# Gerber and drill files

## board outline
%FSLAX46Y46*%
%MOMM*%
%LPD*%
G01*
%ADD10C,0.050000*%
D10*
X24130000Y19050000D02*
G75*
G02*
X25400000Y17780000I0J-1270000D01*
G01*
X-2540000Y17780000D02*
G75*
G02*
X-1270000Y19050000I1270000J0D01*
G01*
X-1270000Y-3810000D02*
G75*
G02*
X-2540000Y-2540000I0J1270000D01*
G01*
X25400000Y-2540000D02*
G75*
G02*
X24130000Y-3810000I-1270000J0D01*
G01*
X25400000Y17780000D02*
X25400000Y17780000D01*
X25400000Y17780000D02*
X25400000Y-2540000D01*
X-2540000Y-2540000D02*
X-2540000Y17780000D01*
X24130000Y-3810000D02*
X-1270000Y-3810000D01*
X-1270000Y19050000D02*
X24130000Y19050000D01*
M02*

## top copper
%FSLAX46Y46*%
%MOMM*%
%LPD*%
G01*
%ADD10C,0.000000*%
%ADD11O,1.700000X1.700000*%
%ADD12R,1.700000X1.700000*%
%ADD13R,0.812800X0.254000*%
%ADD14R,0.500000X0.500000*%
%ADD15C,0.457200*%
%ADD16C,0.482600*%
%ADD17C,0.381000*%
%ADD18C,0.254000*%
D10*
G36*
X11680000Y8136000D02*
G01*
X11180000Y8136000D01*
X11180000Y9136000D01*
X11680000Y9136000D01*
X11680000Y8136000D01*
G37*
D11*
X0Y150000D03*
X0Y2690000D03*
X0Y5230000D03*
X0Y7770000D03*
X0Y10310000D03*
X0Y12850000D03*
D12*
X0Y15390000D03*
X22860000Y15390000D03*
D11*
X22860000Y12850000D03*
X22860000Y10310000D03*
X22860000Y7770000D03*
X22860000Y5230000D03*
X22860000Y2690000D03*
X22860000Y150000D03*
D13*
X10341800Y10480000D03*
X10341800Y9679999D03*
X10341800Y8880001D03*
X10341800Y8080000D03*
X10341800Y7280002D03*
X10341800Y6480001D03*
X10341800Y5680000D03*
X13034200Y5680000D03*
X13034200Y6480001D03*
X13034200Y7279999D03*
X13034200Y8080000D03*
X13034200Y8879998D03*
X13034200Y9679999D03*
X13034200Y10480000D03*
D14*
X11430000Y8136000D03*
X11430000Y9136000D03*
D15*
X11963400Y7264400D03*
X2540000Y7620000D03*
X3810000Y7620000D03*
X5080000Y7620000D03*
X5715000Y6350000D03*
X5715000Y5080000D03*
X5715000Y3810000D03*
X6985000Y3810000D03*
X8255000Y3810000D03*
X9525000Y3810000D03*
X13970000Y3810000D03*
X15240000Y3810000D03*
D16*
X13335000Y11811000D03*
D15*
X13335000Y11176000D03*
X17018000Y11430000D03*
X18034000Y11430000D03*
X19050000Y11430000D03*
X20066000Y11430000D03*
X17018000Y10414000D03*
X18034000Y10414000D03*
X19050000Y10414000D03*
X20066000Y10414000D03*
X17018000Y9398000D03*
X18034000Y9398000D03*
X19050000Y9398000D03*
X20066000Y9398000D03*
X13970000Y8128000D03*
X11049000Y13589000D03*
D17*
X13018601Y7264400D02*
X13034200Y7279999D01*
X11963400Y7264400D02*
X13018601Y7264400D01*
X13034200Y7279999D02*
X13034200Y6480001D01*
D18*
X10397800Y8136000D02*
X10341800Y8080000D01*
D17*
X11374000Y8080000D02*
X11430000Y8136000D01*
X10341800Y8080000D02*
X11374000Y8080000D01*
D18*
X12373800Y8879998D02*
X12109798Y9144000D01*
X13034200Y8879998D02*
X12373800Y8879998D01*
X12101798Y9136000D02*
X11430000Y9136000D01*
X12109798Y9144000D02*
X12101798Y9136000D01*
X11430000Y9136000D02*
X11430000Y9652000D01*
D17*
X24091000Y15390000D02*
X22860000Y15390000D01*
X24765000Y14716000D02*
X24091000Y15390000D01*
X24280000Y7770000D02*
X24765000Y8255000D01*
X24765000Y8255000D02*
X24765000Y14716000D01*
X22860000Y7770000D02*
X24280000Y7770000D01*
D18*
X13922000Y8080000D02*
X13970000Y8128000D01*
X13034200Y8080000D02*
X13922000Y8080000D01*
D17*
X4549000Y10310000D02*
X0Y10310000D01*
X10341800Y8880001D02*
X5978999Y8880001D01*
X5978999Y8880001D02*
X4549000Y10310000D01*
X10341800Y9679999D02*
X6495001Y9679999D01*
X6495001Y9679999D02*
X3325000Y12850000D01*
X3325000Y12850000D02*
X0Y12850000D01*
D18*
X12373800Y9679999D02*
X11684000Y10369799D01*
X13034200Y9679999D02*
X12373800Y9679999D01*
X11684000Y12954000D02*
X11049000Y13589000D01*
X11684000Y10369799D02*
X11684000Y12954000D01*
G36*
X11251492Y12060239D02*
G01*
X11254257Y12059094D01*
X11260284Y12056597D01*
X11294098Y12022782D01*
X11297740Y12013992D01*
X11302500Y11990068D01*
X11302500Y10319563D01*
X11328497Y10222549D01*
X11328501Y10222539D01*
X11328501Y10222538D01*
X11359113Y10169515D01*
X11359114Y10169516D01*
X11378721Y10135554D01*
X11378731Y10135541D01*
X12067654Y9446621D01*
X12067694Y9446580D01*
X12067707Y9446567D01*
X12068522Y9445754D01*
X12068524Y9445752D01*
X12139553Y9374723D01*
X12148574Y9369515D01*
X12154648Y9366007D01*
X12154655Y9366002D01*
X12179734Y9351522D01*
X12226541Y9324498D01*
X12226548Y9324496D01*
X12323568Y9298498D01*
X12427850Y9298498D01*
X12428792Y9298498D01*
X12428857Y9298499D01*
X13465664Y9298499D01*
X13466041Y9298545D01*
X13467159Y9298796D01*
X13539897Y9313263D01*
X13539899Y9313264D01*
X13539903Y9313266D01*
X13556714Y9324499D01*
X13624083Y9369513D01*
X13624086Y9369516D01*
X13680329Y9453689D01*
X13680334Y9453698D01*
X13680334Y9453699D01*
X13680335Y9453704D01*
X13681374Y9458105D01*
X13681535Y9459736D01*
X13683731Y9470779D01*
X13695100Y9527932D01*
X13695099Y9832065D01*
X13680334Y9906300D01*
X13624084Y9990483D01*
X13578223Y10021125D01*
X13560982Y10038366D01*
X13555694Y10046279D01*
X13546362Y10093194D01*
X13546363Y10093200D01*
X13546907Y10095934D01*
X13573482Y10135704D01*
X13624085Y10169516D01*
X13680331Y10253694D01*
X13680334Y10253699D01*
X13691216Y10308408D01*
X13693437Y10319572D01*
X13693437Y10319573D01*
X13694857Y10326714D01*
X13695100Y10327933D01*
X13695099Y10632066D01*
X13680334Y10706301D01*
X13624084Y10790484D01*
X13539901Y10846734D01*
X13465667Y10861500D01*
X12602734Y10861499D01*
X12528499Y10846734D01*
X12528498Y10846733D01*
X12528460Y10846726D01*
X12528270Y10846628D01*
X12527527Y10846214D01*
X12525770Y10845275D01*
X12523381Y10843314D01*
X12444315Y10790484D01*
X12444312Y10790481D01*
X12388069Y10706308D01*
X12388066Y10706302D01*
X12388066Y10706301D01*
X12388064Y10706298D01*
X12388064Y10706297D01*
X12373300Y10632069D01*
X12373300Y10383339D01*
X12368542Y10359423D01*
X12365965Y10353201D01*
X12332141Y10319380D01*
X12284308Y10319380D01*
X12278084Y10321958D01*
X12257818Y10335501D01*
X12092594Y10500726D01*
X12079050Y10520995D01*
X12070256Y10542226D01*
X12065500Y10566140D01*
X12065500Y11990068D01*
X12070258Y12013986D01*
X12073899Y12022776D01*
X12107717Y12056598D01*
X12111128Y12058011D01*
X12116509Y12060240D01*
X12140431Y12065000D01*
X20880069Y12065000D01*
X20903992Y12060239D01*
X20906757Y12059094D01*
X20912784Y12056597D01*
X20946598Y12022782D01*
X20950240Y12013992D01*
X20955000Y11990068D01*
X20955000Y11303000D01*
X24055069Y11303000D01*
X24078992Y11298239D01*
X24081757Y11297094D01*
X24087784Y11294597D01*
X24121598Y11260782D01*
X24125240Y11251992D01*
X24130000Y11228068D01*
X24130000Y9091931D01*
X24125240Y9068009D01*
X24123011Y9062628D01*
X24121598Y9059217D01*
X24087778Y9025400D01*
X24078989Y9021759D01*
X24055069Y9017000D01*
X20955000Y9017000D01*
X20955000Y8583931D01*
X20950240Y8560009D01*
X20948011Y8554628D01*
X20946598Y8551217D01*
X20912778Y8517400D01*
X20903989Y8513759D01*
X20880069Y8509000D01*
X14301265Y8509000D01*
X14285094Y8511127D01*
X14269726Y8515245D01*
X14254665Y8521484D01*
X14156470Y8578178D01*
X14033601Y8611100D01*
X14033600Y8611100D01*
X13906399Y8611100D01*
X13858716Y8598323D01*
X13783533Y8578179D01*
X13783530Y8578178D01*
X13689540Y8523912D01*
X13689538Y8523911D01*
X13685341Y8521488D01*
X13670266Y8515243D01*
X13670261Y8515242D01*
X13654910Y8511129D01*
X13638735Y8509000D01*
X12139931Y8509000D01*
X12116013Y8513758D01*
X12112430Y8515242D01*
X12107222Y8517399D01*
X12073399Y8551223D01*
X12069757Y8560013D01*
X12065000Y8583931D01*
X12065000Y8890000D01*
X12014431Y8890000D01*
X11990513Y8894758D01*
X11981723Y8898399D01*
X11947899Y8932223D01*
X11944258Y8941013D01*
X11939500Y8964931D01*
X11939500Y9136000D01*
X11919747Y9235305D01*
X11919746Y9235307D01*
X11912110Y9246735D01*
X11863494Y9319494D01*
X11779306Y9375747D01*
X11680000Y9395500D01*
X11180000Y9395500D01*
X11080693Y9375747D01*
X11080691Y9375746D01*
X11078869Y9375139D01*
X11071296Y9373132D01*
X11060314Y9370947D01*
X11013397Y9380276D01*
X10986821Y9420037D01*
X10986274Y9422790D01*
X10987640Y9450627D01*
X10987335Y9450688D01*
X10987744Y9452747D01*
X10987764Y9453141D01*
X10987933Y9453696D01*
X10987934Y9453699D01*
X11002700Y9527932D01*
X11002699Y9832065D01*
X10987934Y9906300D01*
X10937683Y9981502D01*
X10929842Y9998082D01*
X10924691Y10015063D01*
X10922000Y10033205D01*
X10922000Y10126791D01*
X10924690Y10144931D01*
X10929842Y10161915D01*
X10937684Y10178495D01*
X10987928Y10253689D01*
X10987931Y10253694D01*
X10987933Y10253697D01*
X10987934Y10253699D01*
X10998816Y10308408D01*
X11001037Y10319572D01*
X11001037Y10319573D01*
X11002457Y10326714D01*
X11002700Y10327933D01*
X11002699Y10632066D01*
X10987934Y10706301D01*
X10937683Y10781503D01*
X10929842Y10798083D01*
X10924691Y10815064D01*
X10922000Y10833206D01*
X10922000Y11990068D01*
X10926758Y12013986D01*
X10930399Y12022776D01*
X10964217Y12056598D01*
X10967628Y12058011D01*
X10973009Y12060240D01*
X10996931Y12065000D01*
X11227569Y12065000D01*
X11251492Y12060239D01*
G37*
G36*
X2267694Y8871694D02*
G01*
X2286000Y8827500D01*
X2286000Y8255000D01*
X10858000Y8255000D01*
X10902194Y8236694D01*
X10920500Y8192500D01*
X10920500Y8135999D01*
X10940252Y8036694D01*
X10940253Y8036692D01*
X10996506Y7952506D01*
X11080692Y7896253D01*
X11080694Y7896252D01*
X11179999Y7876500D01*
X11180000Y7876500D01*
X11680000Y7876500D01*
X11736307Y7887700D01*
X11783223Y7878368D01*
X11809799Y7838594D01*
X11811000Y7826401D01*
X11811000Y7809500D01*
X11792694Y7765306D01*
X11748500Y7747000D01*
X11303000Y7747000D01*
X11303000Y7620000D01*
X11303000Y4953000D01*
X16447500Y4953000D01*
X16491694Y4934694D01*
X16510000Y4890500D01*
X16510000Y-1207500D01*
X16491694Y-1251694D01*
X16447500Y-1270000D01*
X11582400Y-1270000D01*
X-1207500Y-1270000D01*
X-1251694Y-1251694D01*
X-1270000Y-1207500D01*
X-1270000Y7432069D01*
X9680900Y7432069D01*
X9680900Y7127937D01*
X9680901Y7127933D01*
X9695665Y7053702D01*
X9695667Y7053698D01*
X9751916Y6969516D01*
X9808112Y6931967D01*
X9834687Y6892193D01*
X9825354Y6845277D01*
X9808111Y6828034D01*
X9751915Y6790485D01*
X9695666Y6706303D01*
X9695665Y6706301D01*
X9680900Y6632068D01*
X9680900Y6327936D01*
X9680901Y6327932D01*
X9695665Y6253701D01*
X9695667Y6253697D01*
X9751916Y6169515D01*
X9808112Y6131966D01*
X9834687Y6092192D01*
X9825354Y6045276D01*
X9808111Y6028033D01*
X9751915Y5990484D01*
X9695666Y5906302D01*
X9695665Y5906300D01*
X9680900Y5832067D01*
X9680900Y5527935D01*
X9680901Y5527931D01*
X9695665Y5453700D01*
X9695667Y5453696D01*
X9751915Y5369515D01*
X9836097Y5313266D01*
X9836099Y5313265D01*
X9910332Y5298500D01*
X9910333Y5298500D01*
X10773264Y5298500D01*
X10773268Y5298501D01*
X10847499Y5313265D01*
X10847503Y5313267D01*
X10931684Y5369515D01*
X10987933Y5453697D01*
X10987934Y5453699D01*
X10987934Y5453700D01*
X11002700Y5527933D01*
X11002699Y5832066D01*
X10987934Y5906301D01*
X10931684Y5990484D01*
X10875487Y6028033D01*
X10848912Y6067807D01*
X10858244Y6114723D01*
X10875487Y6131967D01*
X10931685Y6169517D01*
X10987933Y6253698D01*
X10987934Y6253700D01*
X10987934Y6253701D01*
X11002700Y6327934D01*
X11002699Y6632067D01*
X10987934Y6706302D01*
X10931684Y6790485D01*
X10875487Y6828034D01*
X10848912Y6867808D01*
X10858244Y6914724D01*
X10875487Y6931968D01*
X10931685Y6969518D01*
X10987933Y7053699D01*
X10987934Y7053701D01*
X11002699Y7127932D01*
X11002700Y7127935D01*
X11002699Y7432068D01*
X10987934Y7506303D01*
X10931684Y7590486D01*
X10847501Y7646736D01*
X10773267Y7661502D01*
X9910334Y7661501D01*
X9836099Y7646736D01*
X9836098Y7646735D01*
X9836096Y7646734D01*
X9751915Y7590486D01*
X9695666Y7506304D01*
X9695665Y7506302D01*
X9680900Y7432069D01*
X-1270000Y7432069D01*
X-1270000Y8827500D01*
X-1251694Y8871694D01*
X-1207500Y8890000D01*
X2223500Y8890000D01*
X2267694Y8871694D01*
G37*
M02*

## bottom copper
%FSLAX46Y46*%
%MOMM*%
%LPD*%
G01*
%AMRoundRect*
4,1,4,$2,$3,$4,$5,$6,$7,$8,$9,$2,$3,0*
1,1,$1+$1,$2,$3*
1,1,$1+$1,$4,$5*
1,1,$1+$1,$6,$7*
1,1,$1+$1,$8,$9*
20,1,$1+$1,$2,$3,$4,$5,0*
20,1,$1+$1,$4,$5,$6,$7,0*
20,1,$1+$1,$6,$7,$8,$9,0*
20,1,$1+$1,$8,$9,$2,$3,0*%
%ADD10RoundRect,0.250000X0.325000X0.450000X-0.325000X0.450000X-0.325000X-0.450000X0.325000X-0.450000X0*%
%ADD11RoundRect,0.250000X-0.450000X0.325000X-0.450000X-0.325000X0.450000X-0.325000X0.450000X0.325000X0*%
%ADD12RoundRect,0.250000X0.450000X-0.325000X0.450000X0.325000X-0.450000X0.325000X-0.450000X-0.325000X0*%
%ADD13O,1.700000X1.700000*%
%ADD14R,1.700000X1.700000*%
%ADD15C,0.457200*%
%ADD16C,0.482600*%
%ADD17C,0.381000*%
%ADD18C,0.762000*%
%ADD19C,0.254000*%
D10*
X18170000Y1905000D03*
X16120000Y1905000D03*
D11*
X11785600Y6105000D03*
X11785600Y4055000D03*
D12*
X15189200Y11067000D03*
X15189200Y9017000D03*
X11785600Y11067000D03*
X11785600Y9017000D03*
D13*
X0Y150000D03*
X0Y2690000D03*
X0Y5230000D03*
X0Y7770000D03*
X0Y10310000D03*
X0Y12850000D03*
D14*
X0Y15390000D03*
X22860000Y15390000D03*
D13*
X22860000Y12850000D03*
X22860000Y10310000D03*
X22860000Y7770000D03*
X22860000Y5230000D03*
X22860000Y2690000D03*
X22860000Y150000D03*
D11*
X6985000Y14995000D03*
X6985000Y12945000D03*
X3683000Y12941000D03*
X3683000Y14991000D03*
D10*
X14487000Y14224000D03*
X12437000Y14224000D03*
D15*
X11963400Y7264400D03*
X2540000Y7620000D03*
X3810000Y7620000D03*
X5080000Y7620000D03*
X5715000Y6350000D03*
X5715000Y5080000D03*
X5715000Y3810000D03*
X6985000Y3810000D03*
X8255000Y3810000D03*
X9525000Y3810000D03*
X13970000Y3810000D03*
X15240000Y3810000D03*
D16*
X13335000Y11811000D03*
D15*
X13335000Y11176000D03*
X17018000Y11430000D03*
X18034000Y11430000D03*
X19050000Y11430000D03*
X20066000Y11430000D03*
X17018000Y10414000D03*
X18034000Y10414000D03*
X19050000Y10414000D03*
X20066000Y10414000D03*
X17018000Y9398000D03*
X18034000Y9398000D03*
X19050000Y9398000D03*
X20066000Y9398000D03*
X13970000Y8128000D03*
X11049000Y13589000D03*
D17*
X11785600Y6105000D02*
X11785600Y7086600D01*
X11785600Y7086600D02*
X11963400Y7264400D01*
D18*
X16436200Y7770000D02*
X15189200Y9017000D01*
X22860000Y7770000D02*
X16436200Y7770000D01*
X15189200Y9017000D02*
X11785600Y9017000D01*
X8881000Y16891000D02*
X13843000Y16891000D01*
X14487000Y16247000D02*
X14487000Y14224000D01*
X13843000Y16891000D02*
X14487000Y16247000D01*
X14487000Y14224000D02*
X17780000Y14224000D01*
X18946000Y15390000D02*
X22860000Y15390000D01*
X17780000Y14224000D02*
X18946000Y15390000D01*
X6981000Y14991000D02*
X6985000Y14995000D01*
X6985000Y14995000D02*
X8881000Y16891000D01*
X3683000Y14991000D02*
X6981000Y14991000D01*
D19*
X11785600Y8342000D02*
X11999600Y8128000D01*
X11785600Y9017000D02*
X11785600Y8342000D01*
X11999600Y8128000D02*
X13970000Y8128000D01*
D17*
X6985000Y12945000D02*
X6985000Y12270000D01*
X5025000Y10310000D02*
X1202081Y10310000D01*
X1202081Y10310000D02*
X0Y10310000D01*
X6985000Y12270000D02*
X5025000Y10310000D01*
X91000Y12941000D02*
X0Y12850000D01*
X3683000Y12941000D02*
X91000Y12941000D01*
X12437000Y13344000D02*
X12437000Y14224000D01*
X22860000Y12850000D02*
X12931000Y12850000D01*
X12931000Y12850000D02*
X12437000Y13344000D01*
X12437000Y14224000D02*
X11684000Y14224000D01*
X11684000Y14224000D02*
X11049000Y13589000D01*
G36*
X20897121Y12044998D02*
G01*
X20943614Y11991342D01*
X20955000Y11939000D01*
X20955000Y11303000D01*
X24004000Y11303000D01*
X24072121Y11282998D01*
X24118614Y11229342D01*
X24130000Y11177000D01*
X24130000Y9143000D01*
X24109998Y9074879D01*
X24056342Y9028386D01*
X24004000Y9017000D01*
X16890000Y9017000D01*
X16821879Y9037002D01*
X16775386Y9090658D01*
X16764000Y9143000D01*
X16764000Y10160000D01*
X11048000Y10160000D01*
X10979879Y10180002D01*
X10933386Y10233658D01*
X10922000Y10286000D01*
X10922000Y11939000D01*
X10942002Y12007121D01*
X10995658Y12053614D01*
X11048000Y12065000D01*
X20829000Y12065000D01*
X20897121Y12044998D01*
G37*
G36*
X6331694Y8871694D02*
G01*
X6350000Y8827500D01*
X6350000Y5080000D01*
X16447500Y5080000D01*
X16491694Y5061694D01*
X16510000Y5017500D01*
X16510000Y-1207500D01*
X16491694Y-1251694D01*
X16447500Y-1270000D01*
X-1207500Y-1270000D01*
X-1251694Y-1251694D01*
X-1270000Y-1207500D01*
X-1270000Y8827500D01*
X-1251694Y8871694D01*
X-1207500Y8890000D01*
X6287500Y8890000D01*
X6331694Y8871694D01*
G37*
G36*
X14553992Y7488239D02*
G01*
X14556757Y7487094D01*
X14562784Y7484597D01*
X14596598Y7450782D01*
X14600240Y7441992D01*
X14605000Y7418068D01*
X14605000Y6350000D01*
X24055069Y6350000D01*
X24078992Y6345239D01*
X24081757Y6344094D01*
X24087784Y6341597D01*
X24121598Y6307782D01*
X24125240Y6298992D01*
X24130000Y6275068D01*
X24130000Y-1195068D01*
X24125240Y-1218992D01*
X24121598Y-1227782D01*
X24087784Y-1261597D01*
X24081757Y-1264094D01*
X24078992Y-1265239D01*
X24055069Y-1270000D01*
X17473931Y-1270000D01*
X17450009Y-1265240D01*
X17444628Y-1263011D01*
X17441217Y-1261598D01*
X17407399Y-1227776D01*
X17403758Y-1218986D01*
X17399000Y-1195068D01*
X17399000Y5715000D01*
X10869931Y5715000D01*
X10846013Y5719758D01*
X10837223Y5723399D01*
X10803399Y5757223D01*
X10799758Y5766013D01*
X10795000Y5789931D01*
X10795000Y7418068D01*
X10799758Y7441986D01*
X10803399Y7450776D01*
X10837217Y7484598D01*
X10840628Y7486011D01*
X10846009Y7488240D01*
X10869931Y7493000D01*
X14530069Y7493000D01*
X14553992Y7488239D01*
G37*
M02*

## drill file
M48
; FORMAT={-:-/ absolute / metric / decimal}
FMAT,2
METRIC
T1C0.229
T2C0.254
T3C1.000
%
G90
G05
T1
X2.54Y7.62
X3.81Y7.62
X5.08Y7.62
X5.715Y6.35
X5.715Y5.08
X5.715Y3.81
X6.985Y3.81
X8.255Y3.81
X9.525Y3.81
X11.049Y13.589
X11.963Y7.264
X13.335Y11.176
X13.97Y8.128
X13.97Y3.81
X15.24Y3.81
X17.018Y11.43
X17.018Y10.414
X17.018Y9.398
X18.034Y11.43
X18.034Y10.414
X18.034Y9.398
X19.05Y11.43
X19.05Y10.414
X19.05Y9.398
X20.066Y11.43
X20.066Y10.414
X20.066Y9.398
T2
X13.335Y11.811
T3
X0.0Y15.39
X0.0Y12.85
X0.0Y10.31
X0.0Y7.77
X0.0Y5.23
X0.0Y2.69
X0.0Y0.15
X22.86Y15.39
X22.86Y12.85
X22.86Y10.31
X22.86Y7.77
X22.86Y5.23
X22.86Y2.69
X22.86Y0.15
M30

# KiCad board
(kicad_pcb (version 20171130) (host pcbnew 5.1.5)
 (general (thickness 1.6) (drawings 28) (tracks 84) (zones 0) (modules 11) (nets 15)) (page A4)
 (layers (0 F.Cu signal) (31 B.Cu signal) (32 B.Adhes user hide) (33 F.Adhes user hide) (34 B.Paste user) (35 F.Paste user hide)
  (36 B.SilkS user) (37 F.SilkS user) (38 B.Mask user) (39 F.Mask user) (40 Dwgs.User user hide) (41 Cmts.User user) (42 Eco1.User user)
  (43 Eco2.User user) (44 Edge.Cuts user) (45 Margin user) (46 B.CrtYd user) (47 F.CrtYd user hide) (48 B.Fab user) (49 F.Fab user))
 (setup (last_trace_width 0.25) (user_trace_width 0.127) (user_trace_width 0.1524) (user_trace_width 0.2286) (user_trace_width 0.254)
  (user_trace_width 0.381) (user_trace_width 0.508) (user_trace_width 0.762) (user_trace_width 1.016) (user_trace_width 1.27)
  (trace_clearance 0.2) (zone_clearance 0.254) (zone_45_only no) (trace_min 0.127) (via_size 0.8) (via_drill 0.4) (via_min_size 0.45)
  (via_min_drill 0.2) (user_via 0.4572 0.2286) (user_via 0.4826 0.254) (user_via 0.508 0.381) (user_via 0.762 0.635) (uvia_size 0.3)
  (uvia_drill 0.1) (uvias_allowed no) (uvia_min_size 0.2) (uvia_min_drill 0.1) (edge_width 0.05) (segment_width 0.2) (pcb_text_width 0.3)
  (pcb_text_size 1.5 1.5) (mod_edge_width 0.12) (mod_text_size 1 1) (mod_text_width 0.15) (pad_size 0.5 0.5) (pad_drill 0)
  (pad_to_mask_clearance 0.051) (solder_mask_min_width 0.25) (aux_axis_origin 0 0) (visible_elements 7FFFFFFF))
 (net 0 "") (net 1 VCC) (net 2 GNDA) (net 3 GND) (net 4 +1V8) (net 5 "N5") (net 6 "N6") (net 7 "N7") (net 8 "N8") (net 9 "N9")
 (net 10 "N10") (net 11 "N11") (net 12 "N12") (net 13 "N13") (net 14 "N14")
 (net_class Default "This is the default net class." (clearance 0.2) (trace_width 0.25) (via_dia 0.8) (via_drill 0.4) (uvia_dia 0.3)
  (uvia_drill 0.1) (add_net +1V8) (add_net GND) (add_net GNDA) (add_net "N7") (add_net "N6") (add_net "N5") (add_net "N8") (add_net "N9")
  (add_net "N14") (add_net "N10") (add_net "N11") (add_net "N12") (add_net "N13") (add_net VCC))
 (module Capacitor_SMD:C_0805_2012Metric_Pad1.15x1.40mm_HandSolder (layer B.Cu) (at 17.145 -1.905 180)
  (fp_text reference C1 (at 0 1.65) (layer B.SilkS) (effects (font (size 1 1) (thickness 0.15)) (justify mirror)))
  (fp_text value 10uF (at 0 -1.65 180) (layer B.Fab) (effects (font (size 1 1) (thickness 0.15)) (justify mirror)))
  (pad 1 smd roundrect (at -1.025 0 180) (size 1.15 1.4) (layers B.Cu B.Paste B.Mask) (roundrect_rratio 0.217391) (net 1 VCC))
  (pad 2 smd roundrect (at 1.025 0 180) (size 1.15 1.4) (layers B.Cu B.Paste B.Mask) (roundrect_rratio 0.217391) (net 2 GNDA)))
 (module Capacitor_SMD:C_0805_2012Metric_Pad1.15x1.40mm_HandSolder (layer B.Cu) (at 11.7856 -5.08 270)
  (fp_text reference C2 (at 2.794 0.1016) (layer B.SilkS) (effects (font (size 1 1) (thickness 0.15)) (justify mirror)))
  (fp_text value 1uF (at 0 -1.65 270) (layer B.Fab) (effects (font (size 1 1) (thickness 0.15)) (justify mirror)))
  (pad 1 smd roundrect (at -1.025 0 270) (size 1.15 1.4) (layers B.Cu B.Paste B.Mask) (roundrect_rratio 0.217391) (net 1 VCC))
  (pad 2 smd roundrect (at 1.025 0 270) (size 1.15 1.4) (layers B.Cu B.Paste B.Mask) (roundrect_rratio 0.217391) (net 2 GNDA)))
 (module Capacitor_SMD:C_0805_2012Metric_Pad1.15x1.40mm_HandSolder (layer B.Cu) (at 15.1892 -10.042 90)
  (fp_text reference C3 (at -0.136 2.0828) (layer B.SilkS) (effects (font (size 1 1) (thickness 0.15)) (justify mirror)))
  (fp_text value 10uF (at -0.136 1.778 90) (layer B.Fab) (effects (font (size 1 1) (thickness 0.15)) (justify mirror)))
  (pad 2 smd roundrect (at 1.025 0 90) (size 1.15 1.4) (layers B.Cu B.Paste B.Mask) (roundrect_rratio 0.217391) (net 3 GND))
  (pad 1 smd roundrect (at -1.025 0 90) (size 1.15 1.4) (layers B.Cu B.Paste B.Mask) (roundrect_rratio 0.217391) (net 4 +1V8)))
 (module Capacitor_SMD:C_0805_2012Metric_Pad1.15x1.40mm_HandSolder (layer B.Cu) (at 11.7856 -10.042 90)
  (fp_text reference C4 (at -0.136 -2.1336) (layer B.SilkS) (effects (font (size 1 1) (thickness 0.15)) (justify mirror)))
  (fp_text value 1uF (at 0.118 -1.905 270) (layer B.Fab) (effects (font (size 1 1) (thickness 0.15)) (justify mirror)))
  (pad 2 smd roundrect (at 1.025 0 90) (size 1.15 1.4) (layers B.Cu B.Paste B.Mask) (roundrect_rratio 0.217391) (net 3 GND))
  (pad 1 smd roundrect (at -1.025 0 90) (size 1.15 1.4) (layers B.Cu B.Paste B.Mask) (roundrect_rratio 0.217391) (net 4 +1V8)))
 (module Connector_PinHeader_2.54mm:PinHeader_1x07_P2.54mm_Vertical (layer F.Cu) (at 0 -15.39)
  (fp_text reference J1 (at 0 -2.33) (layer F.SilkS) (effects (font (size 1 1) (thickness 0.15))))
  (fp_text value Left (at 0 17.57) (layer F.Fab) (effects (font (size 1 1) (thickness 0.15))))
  (pad 7 thru_hole oval (at 0 15.24) (size 1.7 1.7) (drill 1) (layers *.Cu *.Mask) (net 2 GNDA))
  (pad 6 thru_hole oval (at 0 12.7) (size 1.7 1.7) (drill 1) (layers *.Cu *.Mask) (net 2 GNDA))
  (pad 5 thru_hole oval (at 0 10.16) (size 1.7 1.7) (drill 1) (layers *.Cu *.Mask) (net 2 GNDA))
  (pad 4 thru_hole oval (at 0 7.62) (size 1.7 1.7) (drill 1) (layers *.Cu *.Mask) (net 2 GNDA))
  (pad 3 thru_hole oval (at 0 5.08) (size 1.7 1.7) (drill 1) (layers *.Cu *.Mask) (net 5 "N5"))
  (pad 2 thru_hole oval (at 0 2.54) (size 1.7 1.7) (drill 1) (layers *.Cu *.Mask) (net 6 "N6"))
  (pad 1 thru_hole rect (at 0 0) (size 1.7 1.7) (drill 1) (layers *.Cu *.Mask) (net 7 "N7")))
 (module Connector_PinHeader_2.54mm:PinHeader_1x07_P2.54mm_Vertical (layer F.Cu) (at 22.86 -15.39)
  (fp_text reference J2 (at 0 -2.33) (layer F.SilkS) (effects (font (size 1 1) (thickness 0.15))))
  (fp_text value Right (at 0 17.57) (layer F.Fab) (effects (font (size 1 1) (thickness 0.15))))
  (pad 1 thru_hole rect (at 0 0) (size 1.7 1.7) (drill 1) (layers *.Cu *.Mask) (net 4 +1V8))
  (pad 2 thru_hole oval (at 0 2.54) (size 1.7 1.7) (drill 1) (layers *.Cu *.Mask) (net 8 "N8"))
  (pad 3 thru_hole oval (at 0 5.08) (size 1.7 1.7) (drill 1) (layers *.Cu *.Mask) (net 3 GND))
  (pad 4 thru_hole oval (at 0 7.62) (size 1.7 1.7) (drill 1) (layers *.Cu *.Mask) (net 4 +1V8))
  (pad 5 thru_hole oval (at 0 10.16) (size 1.7 1.7) (drill 1) (layers *.Cu *.Mask) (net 1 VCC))
  (pad 6 thru_hole oval (at 0 12.7) (size 1.7 1.7) (drill 1) (layers *.Cu *.Mask) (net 1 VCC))
  (pad 7 thru_hole oval (at 0 15.24) (size 1.7 1.7) (drill 1) (layers *.Cu *.Mask) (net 1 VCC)))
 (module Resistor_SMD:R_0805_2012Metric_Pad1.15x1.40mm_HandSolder (layer B.Cu) (at 6.985 -13.97 270)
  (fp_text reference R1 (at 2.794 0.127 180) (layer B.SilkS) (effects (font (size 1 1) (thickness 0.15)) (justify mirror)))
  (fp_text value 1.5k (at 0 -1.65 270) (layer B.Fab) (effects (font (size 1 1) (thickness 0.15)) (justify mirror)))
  (pad 1 smd roundrect (at -1.025 0 270) (size 1.15 1.4) (layers B.Cu B.Paste B.Mask) (roundrect_rratio 0.217391) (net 4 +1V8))
  (pad 2 smd roundrect (at 1.025 0 270) (size 1.15 1.4) (layers B.Cu B.Paste B.Mask) (roundrect_rratio 0.217391) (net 5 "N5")))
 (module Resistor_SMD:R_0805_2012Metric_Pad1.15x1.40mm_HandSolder (layer B.Cu) (at 3.683 -13.966 270)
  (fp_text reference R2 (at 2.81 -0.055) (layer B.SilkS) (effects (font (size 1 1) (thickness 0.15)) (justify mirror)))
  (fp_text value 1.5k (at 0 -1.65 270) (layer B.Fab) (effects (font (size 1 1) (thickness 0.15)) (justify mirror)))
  (pad 2 smd roundrect (at 1.025 0 270) (size 1.15 1.4) (layers B.Cu B.Paste B.Mask) (roundrect_rratio 0.217391) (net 6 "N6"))
  (pad 1 smd roundrect (at -1.025 0 270) (size 1.15 1.4) (layers B.Cu B.Paste B.Mask) (roundrect_rratio 0.217391) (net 4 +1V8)))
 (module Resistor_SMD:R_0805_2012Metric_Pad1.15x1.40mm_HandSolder (layer B.Cu) (at 13.462 -14.224 180)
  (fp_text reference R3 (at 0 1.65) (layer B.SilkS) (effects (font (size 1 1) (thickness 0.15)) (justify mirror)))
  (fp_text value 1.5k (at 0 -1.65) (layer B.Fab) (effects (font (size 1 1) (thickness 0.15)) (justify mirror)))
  (pad 1 smd roundrect (at -1.025 0 180) (size 1.15 1.4) (layers B.Cu B.Paste B.Mask) (roundrect_rratio 0.217391) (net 4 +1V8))
  (pad 2 smd roundrect (at 1.025 0 180) (size 1.15 1.4) (layers B.Cu B.Paste B.Mask) (roundrect_rratio 0.217391) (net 8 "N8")))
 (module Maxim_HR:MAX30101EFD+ (layer F.Cu) (at 11.688 -8.08)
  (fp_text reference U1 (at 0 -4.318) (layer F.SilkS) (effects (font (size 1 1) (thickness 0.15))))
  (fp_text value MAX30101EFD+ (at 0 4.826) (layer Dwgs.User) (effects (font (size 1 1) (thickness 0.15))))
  (pad 1 smd rect (at -1.3462 -2.4) (size 0.8128 0.254) (layers F.Cu F.Paste F.Mask) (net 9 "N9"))
  (pad 2 smd rect (at -1.3462 -1.599999) (size 0.8128 0.254) (layers F.Cu F.Paste F.Mask) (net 6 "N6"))
  (pad 3 smd rect (at -1.3462 -0.800001) (size 0.8128 0.254) (layers F.Cu F.Paste F.Mask) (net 5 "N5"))
  (pad 4 smd rect (at -1.3462 0) (size 0.8128 0.254) (layers F.Cu F.Paste F.Mask) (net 2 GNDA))
  (pad 5 smd rect (at -1.3462 0.799998) (size 0.8128 0.254) (layers F.Cu F.Paste F.Mask) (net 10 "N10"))
  (pad 6 smd rect (at -1.3462 1.599999) (size 0.8128 0.254) (layers F.Cu F.Paste F.Mask) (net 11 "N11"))
  (pad 7 smd rect (at -1.3462 2.4) (size 0.8128 0.254) (layers F.Cu F.Paste F.Mask) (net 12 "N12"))
  (pad 8 smd rect (at 1.3462 2.4) (size 0.8128 0.254) (layers F.Cu F.Paste F.Mask) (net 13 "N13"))
  (pad 9 smd rect (at 1.3462 1.599999) (size 0.8128 0.254) (layers F.Cu F.Paste F.Mask) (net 1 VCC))
  (pad 10 smd rect (at 1.3462 0.800001) (size 0.8128 0.254) (layers F.Cu F.Paste F.Mask) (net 1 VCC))
  (pad 11 smd rect (at 1.3462 0) (size 0.8128 0.254) (layers F.Cu F.Paste F.Mask) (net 4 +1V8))
  (pad 12 smd rect (at 1.3462 -0.799998) (size 0.8128 0.254) (layers F.Cu F.Paste F.Mask) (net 3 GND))
  (pad 13 smd rect (at 1.3462 -1.599999) (size 0.8128 0.254) (layers F.Cu F.Paste F.Mask) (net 8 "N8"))
  (pad 14 smd rect (at 1.3462 -2.4) (size 0.8128 0.254) (layers F.Cu F.Paste F.Mask) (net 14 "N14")))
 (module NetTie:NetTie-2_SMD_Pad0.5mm (layer F.Cu) (at 11.43 -8.636 90)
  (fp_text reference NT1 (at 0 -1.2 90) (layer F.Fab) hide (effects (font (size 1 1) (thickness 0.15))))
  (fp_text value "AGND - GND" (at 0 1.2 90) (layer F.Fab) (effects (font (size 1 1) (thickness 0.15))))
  (fp_poly (pts (xy -0.5 -0.25) (xy 0.5 -0.25) (xy 0.5 0.25) (xy -0.5 0.25)) (layer F.Cu) (width 0))
  (pad 1 smd rect (at -0.5 0 90) (size 0.5 0.5) (layers F.Cu) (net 2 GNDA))
  (pad 2 smd rect (at 0.5 0 90) (size 0.5 0.5) (layers F.Cu) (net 3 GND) (zone_connect 2) (thermal_width 1.27) (thermal_gap 0.127)))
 (gr_arc (start 24.13 -17.78) (end 25.4 -17.78) (angle -90) (layer Edge.Cuts) (width 0.05))
 (gr_arc (start -1.27 -17.78) (end -1.27 -19.05) (angle -90) (layer Edge.Cuts) (width 0.05))
 (gr_arc (start -1.27 2.54) (end -2.54 2.54) (angle -90) (layer Edge.Cuts) (width 0.05))
 (gr_arc (start 24.13 2.54) (end 24.13 3.81) (angle -90) (layer Edge.Cuts) (width 0.05))
 (gr_line (start 25.4 -17.78) (end 25.4 -17.78) (layer Edge.Cuts) (width 0.05))
 (gr_line (start 25.4 -17.78) (end 25.4 2.54) (layer Edge.Cuts) (width 0.05))
 (gr_line (start -2.54 2.54) (end -2.54 -17.78) (layer Edge.Cuts) (width 0.05))
 (gr_line (start 24.13 3.81) (end -1.27 3.81) (layer Edge.Cuts) (width 0.05))
 (gr_line (start -1.27 -19.05) (end 24.13 -19.05) (layer Edge.Cuts) (width 0.05))
 (via (at 11.9634 -7.2644) (size 0.4572) (drill 0.2286) (layers F.Cu B.Cu) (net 1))
 (segment (start 11.7856 -6.105) (end 11.7856 -7.0866) (width 0.381) (layer B.Cu) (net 1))
 (segment (start 11.7856 -7.0866) (end 11.9634 -7.2644) (width 0.381) (layer B.Cu) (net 1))
 (segment (start 13.018601 -7.2644) (end 13.0342 -7.279999) (width 0.381) (layer F.Cu) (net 1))
 (segment (start 11.9634 -7.2644) (end 13.018601 -7.2644) (width 0.381) (layer F.Cu) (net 1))
 (segment (start 13.0342 -7.279999) (end 13.0342 -6.480001) (width 0.381) (layer F.Cu) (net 1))
 (segment (start 10.3978 -8.136) (end 10.3418 -8.08) (width 0.254) (layer F.Cu) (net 2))
 (via (at 2.54 -7.62) (size 0.4572) (drill 0.2286) (layers F.Cu B.Cu) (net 2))
 (via (at 3.81 -7.62) (size 0.4572) (drill 0.2286) (layers F.Cu B.Cu) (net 2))
 (via (at 5.08 -7.62) (size 0.4572) (drill 0.2286) (layers F.Cu B.Cu) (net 2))
 (via (at 5.715 -6.35) (size 0.4572) (drill 0.2286) (layers F.Cu B.Cu) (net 2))
 (via (at 5.715 -5.08) (size 0.4572) (drill 0.2286) (layers F.Cu B.Cu) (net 2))
 (via (at 5.715 -3.81) (size 0.4572) (drill 0.2286) (layers F.Cu B.Cu) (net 2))
 (via (at 6.985 -3.81) (size 0.4572) (drill 0.2286) (layers F.Cu B.Cu) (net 2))
 (via (at 8.255 -3.81) (size 0.4572) (drill 0.2286) (layers F.Cu B.Cu) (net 2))
 (via (at 9.525 -3.81) (size 0.4572) (drill 0.2286) (layers F.Cu B.Cu) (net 2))
 (via (at 13.97 -3.81) (size 0.4572) (drill 0.2286) (layers F.Cu B.Cu) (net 2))
 (via (at 15.24 -3.81) (size 0.4572) (drill 0.2286) (layers F.Cu B.Cu) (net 2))
 (segment (start 11.374 -8.08) (end 11.43 -8.136) (width 0.381) (layer F.Cu) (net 2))
 (segment (start 10.3418 -8.08) (end 11.374 -8.08) (width 0.381) (layer F.Cu) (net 2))
 (via (at 13.335 -11.811) (size 0.4826) (drill 0.254) (layers F.Cu B.Cu) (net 3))
 (via (at 13.335 -11.176) (size 0.4572) (drill 0.2286) (layers F.Cu B.Cu) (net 3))
 (segment (start 12.3738 -8.879998) (end 12.109798 -9.144) (width 0.254) (layer F.Cu) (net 3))
 (segment (start 13.0342 -8.879998) (end 12.3738 -8.879998) (width 0.254) (layer F.Cu) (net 3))
 (segment (start 12.101798 -9.136) (end 11.43 -9.136) (width 0.254) (layer F.Cu) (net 3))
 (segment (start 12.109798 -9.144) (end 12.101798 -9.136) (width 0.254) (layer F.Cu) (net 3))
 (segment (start 11.43 -9.136) (end 11.43 -9.652) (width 0.254) (layer F.Cu) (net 3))
 (via (at 17.018 -11.43) (size 0.4572) (drill 0.2286) (layers F.Cu B.Cu) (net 3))
 (via (at 18.034 -11.43) (size 0.4572) (drill 0.2286) (layers F.Cu B.Cu) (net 3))
 (via (at 19.05 -11.43) (size 0.4572) (drill 0.2286) (layers F.Cu B.Cu) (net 3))
 (via (at 20.066 -11.43) (size 0.4572) (drill 0.2286) (layers F.Cu B.Cu) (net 3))
 (via (at 17.018 -10.414) (size 0.4572) (drill 0.2286) (layers F.Cu B.Cu) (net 3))
 (via (at 18.034 -10.414) (size 0.4572) (drill 0.2286) (layers F.Cu B.Cu) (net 3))
 (via (at 19.05 -10.414) (size 0.4572) (drill 0.2286) (layers F.Cu B.Cu) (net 3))
 (via (at 20.066 -10.414) (size 0.4572) (drill 0.2286) (layers F.Cu B.Cu) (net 3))
 (via (at 17.018 -9.398) (size 0.4572) (drill 0.2286) (layers F.Cu B.Cu) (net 3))
 (via (at 18.034 -9.398) (size 0.4572) (drill 0.2286) (layers F.Cu B.Cu) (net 3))
 (via (at 19.05 -9.398) (size 0.4572) (drill 0.2286) (layers F.Cu B.Cu) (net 3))
 (via (at 20.066 -9.398) (size 0.4572) (drill 0.2286) (layers F.Cu B.Cu) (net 3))
 (segment (start 16.4362 -7.77) (end 15.1892 -9.017) (width 0.762) (layer B.Cu) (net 4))
 (segment (start 22.86 -7.77) (end 16.4362 -7.77) (width 0.762) (layer B.Cu) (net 4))
 (segment (start 15.1892 -9.017) (end 11.7856 -9.017) (width 0.762) (layer B.Cu) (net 4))
 (segment (start 8.881 -16.891) (end 13.843 -16.891) (width 0.762) (layer B.Cu) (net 4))
 (segment (start 14.487 -16.247) (end 14.487 -14.224) (width 0.762) (layer B.Cu) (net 4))
 (segment (start 13.843 -16.891) (end 14.487 -16.247) (width 0.762) (layer B.Cu) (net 4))
 (segment (start 14.487 -14.224) (end 17.78 -14.224) (width 0.762) (layer B.Cu) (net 4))
 (segment (start 18.946 -15.39) (end 22.86 -15.39) (width 0.762) (layer B.Cu) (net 4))
 (segment (start 17.78 -14.224) (end 18.946 -15.39) (width 0.762) (layer B.Cu) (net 4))
 (segment (start 6.981 -14.991) (end 6.985 -14.995) (width 0.762) (layer B.Cu) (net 4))
 (segment (start 6.985 -14.995) (end 8.881 -16.891) (width 0.762) (layer B.Cu) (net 4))
 (segment (start 3.683 -14.991) (end 6.981 -14.991) (width 0.762) (layer B.Cu) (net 4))
 (segment (start 24.091 -15.39) (end 22.86 -15.39) (width 0.381) (layer F.Cu) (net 4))
 (segment (start 24.765 -14.716) (end 24.091 -15.39) (width 0.381) (layer F.Cu) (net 4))
 (segment (start 24.28 -7.77) (end 24.765 -8.255) (width 0.381) (layer F.Cu) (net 4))
 (segment (start 24.765 -8.255) (end 24.765 -14.716) (width 0.381) (layer F.Cu) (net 4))
 (segment (start 22.86 -7.77) (end 24.28 -7.77) (width 0.381) (layer F.Cu) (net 4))
 (segment (start 11.7856 -8.342) (end 11.9996 -8.128) (width 0.254) (layer B.Cu) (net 4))
 (segment (start 11.7856 -9.017) (end 11.7856 -8.342) (width 0.254) (layer B.Cu) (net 4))
 (via (at 13.97 -8.128) (size 0.4572) (drill 0.2286) (layers F.Cu B.Cu) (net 4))
 (segment (start 11.9996 -8.128) (end 13.97 -8.128) (width 0.254) (layer B.Cu) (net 4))
 (segment (start 13.922 -8.08) (end 13.97 -8.128) (width 0.254) (layer F.Cu) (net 4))
 (segment (start 13.0342 -8.08) (end 13.922 -8.08) (width 0.254) (layer F.Cu) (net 4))
 (segment (start 4.549 -10.31) (end 0 -10.31) (width 0.381) (layer F.Cu) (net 5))
 (segment (start 10.3418 -8.880001) (end 5.978999 -8.880001) (width 0.381) (layer F.Cu) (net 5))
 (segment (start 5.978999 -8.880001) (end 4.549 -10.31) (width 0.381) (layer F.Cu) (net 5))
 (segment (start 6.985 -12.945) (end 6.985 -12.27) (width 0.381) (layer B.Cu) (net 5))
 (segment (start 5.025 -10.31) (end 1.202081 -10.31) (width 0.381) (layer B.Cu) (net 5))
 (segment (start 1.202081 -10.31) (end 0 -10.31) (width 0.381) (layer B.Cu) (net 5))
 (segment (start 6.985 -12.27) (end 5.025 -10.31) (width 0.381) (layer B.Cu) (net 5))
 (segment (start 10.3418 -9.679999) (end 6.495001 -9.679999) (width 0.381) (layer F.Cu) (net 6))
 (segment (start 6.495001 -9.679999) (end 3.325 -12.85) (width 0.381) (layer F.Cu) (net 6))
 (segment (start 3.325 -12.85) (end 0 -12.85) (width 0.381) (layer F.Cu) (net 6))
 (segment (start 0.091 -12.941) (end 0 -12.85) (width 0.381) (layer B.Cu) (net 6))
 (segment (start 3.683 -12.941) (end 0.091 -12.941) (width 0.381) (layer B.Cu) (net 6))
 (segment (start 12.437 -13.344) (end 12.437 -14.224) (width 0.381) (layer B.Cu) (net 8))
 (segment (start 22.86 -12.85) (end 12.931 -12.85) (width 0.381) (layer B.Cu) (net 8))
 (segment (start 12.931 -12.85) (end 12.437 -13.344) (width 0.381) (layer B.Cu) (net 8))
 (via (at 11.049 -13.589) (size 0.4572) (drill 0.2286) (layers F.Cu B.Cu) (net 8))
 (segment (start 12.437 -14.224) (end 11.684 -14.224) (width 0.381) (layer B.Cu) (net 8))
 (segment (start 11.684 -14.224) (end 11.049 -13.589) (width 0.381) (layer B.Cu) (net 8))
 (segment (start 12.3738 -9.679999) (end 11.684 -10.369799) (width 0.254) (layer F.Cu) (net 8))
 (segment (start 13.0342 -9.679999) (end 12.3738 -9.679999) (width 0.254) (layer F.Cu) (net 8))
 (segment (start 11.684 -12.954) (end 11.049 -13.589) (width 0.254) (layer F.Cu) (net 8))
 (segment (start 11.684 -10.369799) (end 11.684 -12.954) (width 0.254) (layer F.Cu) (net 8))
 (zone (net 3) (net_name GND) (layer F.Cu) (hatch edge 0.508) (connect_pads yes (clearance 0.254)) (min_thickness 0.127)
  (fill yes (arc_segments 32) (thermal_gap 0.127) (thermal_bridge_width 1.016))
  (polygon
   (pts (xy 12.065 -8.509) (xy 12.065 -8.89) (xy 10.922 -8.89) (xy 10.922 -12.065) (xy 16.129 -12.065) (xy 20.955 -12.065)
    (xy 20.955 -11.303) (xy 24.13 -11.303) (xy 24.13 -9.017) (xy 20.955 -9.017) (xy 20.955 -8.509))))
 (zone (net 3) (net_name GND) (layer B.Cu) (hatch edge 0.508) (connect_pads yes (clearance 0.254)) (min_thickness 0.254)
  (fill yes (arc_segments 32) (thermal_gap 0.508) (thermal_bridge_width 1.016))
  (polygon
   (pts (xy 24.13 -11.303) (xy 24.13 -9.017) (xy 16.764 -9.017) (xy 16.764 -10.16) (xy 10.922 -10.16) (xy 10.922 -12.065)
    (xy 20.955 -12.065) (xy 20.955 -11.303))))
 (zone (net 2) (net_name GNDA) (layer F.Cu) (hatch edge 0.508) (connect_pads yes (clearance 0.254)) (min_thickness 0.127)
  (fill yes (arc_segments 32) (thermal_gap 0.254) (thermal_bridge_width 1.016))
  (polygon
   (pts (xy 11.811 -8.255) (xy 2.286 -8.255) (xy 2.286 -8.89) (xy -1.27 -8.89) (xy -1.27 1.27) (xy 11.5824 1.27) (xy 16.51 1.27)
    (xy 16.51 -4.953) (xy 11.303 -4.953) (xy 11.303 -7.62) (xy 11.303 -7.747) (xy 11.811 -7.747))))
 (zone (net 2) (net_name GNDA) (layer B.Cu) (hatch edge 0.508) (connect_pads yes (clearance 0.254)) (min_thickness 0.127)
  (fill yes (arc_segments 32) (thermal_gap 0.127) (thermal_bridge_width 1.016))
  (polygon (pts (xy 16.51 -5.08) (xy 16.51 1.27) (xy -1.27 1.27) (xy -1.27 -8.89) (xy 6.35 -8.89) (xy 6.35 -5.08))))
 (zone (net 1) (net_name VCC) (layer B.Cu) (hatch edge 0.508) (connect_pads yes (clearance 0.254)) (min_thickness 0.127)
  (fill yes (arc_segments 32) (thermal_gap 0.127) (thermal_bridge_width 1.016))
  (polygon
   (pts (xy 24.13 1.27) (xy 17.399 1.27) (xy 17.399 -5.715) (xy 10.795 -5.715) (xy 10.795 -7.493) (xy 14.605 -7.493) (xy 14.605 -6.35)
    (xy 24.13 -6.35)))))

